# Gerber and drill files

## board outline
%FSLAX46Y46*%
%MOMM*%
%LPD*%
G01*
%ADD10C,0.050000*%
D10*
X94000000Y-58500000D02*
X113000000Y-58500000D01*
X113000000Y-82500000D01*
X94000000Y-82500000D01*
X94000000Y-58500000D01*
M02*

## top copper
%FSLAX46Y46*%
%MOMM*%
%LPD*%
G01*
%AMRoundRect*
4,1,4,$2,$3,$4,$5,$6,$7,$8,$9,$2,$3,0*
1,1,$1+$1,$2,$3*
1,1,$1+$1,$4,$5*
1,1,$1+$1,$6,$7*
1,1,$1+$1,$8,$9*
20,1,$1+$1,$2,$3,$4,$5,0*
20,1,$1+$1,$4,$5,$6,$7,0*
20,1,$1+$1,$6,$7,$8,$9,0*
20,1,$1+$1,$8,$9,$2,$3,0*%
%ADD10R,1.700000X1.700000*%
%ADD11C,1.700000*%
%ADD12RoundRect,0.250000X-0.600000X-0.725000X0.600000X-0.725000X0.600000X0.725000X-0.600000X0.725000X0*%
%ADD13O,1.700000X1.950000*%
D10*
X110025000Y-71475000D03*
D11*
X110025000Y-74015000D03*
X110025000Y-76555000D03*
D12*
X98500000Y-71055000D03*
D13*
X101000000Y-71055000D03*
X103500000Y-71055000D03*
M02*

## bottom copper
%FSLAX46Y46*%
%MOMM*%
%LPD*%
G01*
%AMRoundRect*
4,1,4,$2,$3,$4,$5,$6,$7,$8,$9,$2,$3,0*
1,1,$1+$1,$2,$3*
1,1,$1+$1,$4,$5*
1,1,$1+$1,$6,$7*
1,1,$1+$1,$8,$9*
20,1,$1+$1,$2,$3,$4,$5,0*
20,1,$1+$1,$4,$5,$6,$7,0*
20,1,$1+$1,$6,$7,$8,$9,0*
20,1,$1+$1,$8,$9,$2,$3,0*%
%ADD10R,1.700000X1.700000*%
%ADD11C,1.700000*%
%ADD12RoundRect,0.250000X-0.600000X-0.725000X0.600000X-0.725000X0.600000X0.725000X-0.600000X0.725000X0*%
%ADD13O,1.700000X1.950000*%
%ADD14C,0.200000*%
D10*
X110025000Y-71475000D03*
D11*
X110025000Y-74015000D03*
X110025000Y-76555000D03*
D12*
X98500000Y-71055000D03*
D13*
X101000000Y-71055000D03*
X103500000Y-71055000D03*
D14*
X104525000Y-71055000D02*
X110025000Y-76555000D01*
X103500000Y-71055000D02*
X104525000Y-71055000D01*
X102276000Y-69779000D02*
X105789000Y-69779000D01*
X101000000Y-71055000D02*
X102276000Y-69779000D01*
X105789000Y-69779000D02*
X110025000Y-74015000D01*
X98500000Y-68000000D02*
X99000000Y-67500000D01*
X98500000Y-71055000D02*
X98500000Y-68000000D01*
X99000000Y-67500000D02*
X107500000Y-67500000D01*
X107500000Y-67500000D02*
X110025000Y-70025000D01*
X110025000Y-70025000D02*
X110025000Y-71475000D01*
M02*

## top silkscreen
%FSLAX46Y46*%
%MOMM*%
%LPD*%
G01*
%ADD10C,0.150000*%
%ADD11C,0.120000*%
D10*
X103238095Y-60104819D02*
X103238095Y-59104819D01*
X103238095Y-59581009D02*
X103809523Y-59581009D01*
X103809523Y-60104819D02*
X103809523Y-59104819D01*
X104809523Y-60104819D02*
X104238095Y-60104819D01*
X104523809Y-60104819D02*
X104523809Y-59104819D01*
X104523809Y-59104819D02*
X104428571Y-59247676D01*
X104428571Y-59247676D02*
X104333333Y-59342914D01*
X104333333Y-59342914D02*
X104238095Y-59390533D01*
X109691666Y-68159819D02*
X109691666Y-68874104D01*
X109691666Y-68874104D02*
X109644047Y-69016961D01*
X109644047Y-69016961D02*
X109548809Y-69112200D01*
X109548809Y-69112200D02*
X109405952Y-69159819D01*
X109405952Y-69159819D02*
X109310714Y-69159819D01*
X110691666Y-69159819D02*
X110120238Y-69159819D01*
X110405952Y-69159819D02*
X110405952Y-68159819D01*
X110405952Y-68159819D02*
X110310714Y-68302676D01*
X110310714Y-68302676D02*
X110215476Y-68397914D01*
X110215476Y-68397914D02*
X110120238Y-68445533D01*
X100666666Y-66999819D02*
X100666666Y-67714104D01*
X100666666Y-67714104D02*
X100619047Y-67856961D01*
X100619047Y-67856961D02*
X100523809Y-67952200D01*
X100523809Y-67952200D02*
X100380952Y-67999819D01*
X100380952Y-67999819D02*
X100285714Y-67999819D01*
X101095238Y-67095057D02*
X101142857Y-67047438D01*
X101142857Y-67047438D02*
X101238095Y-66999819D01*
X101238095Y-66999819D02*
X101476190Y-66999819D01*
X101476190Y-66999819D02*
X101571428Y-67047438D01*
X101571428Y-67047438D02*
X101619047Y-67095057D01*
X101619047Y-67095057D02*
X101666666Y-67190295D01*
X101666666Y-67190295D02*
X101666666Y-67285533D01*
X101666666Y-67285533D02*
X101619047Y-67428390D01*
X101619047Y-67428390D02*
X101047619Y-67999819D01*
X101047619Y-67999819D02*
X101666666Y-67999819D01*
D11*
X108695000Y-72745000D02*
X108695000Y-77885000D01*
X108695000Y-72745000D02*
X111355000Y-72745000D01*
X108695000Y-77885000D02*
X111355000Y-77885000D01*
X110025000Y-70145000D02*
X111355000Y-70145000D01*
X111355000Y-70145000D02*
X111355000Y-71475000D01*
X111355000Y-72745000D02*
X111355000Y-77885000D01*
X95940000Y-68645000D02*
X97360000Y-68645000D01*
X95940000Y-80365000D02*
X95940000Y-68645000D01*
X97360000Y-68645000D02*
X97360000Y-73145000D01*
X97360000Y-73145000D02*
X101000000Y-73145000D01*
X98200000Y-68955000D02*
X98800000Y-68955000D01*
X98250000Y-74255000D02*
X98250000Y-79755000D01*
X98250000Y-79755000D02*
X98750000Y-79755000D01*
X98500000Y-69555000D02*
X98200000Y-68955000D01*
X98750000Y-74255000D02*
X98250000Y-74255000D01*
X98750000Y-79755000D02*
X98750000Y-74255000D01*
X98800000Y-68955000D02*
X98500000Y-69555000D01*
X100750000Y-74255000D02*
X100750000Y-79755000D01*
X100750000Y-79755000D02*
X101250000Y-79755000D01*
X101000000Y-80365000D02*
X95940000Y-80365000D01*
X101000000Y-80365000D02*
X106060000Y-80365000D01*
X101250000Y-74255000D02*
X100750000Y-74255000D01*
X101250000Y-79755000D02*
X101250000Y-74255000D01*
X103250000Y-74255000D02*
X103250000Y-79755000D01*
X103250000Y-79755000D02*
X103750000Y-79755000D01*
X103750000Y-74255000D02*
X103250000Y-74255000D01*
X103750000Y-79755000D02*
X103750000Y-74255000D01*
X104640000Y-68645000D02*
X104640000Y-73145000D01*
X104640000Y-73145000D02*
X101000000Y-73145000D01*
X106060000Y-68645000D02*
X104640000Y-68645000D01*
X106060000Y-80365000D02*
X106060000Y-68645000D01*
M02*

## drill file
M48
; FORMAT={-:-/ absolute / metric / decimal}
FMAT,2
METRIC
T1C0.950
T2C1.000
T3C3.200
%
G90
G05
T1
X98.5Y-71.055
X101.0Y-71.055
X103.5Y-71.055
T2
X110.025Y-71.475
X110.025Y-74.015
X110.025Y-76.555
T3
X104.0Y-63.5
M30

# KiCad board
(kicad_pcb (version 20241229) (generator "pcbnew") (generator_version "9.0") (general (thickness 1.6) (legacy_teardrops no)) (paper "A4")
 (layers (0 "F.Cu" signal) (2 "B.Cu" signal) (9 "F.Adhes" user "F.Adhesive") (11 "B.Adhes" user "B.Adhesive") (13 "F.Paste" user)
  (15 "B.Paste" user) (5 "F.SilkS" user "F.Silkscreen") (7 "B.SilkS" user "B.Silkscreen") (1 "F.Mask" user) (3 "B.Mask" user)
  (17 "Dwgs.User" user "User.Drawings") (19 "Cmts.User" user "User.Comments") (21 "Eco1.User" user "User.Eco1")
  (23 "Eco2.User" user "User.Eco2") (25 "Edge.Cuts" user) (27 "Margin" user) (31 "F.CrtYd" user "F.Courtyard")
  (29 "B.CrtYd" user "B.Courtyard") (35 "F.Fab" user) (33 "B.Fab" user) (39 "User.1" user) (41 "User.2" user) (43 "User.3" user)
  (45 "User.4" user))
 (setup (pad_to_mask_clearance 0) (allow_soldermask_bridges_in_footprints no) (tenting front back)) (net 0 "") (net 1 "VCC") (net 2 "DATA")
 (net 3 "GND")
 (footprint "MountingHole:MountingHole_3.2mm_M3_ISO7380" (layer "F.Cu") (at 104 63.5)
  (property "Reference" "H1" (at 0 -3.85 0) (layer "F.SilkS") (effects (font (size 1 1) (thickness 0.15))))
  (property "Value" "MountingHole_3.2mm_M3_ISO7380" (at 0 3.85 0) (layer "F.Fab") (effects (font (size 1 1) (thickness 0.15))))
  (pad "" np_thru_hole circle (at 0 0) (size 3.2 3.2) (drill 3.2) (layers "*.Cu" "*.Mask")))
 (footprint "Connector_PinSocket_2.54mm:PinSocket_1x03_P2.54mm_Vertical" (layer "F.Cu") (at 110.025 71.475)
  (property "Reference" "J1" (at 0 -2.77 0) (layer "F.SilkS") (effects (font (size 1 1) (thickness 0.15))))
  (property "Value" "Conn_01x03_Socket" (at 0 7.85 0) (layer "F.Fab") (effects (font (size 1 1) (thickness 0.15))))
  (fp_line (start -1.33 1.27) (end -1.33 6.41) (stroke (width 0.12) (type solid)) (layer "F.SilkS"))
  (fp_line (start -1.33 1.27) (end 1.33 1.27) (stroke (width 0.12) (type solid)) (layer "F.SilkS"))
  (fp_line (start -1.33 6.41) (end 1.33 6.41) (stroke (width 0.12) (type solid)) (layer "F.SilkS"))
  (fp_line (start 0 -1.33) (end 1.33 -1.33) (stroke (width 0.12) (type solid)) (layer "F.SilkS"))
  (fp_line (start 1.33 -1.33) (end 1.33 0) (stroke (width 0.12) (type solid)) (layer "F.SilkS"))
  (fp_line (start 1.33 1.27) (end 1.33 6.41) (stroke (width 0.12) (type solid)) (layer "F.SilkS"))
  (pad "1" thru_hole rect (at 0 0) (size 1.7 1.7) (drill 1) (layers "*.Cu" "*.Mask") (remove_unused_layers no) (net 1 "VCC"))
  (pad "2" thru_hole circle (at 0 2.54) (size 1.7 1.7) (drill 1) (layers "*.Cu" "*.Mask") (remove_unused_layers no) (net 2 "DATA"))
  (pad "3" thru_hole circle (at 0 5.08) (size 1.7 1.7) (drill 1) (layers "*.Cu" "*.Mask") (remove_unused_layers no) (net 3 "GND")))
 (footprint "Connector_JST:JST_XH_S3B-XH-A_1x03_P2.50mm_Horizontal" (layer "F.Cu") (at 98.5 71.055)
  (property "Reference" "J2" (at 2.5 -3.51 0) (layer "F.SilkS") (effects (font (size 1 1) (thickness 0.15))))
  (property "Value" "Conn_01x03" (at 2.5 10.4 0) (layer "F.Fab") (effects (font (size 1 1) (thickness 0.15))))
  (fp_line (start -2.56 -2.41) (end -1.14 -2.41) (stroke (width 0.12) (type solid)) (layer "F.SilkS"))
  (fp_line (start -2.56 9.31) (end -2.56 -2.41) (stroke (width 0.12) (type solid)) (layer "F.SilkS"))
  (fp_line (start -1.14 -2.41) (end -1.14 2.09) (stroke (width 0.12) (type solid)) (layer "F.SilkS"))
  (fp_line (start -1.14 2.09) (end 2.5 2.09) (stroke (width 0.12) (type solid)) (layer "F.SilkS"))
  (fp_line (start -0.3 -2.1) (end 0.3 -2.1) (stroke (width 0.12) (type solid)) (layer "F.SilkS"))
  (fp_line (start -0.25 3.2) (end -0.25 8.7) (stroke (width 0.12) (type solid)) (layer "F.SilkS"))
  (fp_line (start -0.25 8.7) (end 0.25 8.7) (stroke (width 0.12) (type solid)) (layer "F.SilkS"))
  (fp_line (start 0 -1.5) (end -0.3 -2.1) (stroke (width 0.12) (type solid)) (layer "F.SilkS"))
  (fp_line (start 0.25 3.2) (end -0.25 3.2) (stroke (width 0.12) (type solid)) (layer "F.SilkS"))
  (fp_line (start 0.25 8.7) (end 0.25 3.2) (stroke (width 0.12) (type solid)) (layer "F.SilkS"))
  (fp_line (start 0.3 -2.1) (end 0 -1.5) (stroke (width 0.12) (type solid)) (layer "F.SilkS"))
  (fp_line (start 2.25 3.2) (end 2.25 8.7) (stroke (width 0.12) (type solid)) (layer "F.SilkS"))
  (fp_line (start 2.25 8.7) (end 2.75 8.7) (stroke (width 0.12) (type solid)) (layer "F.SilkS"))
  (fp_line (start 2.5 9.31) (end -2.56 9.31) (stroke (width 0.12) (type solid)) (layer "F.SilkS"))
  (fp_line (start 2.5 9.31) (end 7.56 9.31) (stroke (width 0.12) (type solid)) (layer "F.SilkS"))
  (fp_line (start 2.75 3.2) (end 2.25 3.2) (stroke (width 0.12) (type solid)) (layer "F.SilkS"))
  (fp_line (start 2.75 8.7) (end 2.75 3.2) (stroke (width 0.12) (type solid)) (layer "F.SilkS"))
  (fp_line (start 4.75 3.2) (end 4.75 8.7) (stroke (width 0.12) (type solid)) (layer "F.SilkS"))
  (fp_line (start 4.75 8.7) (end 5.25 8.7) (stroke (width 0.12) (type solid)) (layer "F.SilkS"))
  (fp_line (start 5.25 3.2) (end 4.75 3.2) (stroke (width 0.12) (type solid)) (layer "F.SilkS"))
  (fp_line (start 5.25 8.7) (end 5.25 3.2) (stroke (width 0.12) (type solid)) (layer "F.SilkS"))
  (fp_line (start 6.14 -2.41) (end 6.14 2.09) (stroke (width 0.12) (type solid)) (layer "F.SilkS"))
  (fp_line (start 6.14 2.09) (end 2.5 2.09) (stroke (width 0.12) (type solid)) (layer "F.SilkS"))
  (fp_line (start 7.56 -2.41) (end 6.14 -2.41) (stroke (width 0.12) (type solid)) (layer "F.SilkS"))
  (fp_line (start 7.56 9.31) (end 7.56 -2.41) (stroke (width 0.12) (type solid)) (layer "F.SilkS"))
  (pad "1" thru_hole roundrect (at 0 0) (size 1.7 1.95) (drill 0.95) (layers "*.Cu" "*.Mask") (remove_unused_layers no)
   (roundrect_rratio 0.147059) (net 1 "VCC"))
  (pad "2" thru_hole oval (at 2.5 0) (size 1.7 1.95) (drill 0.95) (layers "*.Cu" "*.Mask") (remove_unused_layers no) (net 2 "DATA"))
  (pad "3" thru_hole oval (at 5 0) (size 1.7 1.95) (drill 0.95) (layers "*.Cu" "*.Mask") (remove_unused_layers no) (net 3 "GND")))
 (gr_rect (start 94 58.5) (end 113 82.5) (stroke (width 0.05) (type default)) (fill no) (layer "Edge.Cuts"))
 (segment (start 104.525 71.055) (end 110.025 76.555) (width 0.2) (layer "B.Cu") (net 3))
 (segment (start 103.5 71.055) (end 104.525 71.055) (width 0.2) (layer "B.Cu") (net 3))
 (segment (start 102.276 69.779) (end 105.789 69.779) (width 0.2) (layer "B.Cu") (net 2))
 (segment (start 101 71.055) (end 102.276 69.779) (width 0.2) (layer "B.Cu") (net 2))
 (segment (start 105.789 69.779) (end 110.025 74.015) (width 0.2) (layer "B.Cu") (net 2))
 (segment (start 98.5 68) (end 99 67.5) (width 0.2) (layer "B.Cu") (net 1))
 (segment (start 98.5 71.055) (end 98.5 68) (width 0.2) (layer "B.Cu") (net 1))
 (segment (start 99 67.5) (end 107.5 67.5) (width 0.2) (layer "B.Cu") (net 1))
 (segment (start 107.5 67.5) (end 110.025 70.025) (width 0.2) (layer "B.Cu") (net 1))
 (segment (start 110.025 70.025) (end 110.025 71.475) (width 0.2) (layer "B.Cu") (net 1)))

